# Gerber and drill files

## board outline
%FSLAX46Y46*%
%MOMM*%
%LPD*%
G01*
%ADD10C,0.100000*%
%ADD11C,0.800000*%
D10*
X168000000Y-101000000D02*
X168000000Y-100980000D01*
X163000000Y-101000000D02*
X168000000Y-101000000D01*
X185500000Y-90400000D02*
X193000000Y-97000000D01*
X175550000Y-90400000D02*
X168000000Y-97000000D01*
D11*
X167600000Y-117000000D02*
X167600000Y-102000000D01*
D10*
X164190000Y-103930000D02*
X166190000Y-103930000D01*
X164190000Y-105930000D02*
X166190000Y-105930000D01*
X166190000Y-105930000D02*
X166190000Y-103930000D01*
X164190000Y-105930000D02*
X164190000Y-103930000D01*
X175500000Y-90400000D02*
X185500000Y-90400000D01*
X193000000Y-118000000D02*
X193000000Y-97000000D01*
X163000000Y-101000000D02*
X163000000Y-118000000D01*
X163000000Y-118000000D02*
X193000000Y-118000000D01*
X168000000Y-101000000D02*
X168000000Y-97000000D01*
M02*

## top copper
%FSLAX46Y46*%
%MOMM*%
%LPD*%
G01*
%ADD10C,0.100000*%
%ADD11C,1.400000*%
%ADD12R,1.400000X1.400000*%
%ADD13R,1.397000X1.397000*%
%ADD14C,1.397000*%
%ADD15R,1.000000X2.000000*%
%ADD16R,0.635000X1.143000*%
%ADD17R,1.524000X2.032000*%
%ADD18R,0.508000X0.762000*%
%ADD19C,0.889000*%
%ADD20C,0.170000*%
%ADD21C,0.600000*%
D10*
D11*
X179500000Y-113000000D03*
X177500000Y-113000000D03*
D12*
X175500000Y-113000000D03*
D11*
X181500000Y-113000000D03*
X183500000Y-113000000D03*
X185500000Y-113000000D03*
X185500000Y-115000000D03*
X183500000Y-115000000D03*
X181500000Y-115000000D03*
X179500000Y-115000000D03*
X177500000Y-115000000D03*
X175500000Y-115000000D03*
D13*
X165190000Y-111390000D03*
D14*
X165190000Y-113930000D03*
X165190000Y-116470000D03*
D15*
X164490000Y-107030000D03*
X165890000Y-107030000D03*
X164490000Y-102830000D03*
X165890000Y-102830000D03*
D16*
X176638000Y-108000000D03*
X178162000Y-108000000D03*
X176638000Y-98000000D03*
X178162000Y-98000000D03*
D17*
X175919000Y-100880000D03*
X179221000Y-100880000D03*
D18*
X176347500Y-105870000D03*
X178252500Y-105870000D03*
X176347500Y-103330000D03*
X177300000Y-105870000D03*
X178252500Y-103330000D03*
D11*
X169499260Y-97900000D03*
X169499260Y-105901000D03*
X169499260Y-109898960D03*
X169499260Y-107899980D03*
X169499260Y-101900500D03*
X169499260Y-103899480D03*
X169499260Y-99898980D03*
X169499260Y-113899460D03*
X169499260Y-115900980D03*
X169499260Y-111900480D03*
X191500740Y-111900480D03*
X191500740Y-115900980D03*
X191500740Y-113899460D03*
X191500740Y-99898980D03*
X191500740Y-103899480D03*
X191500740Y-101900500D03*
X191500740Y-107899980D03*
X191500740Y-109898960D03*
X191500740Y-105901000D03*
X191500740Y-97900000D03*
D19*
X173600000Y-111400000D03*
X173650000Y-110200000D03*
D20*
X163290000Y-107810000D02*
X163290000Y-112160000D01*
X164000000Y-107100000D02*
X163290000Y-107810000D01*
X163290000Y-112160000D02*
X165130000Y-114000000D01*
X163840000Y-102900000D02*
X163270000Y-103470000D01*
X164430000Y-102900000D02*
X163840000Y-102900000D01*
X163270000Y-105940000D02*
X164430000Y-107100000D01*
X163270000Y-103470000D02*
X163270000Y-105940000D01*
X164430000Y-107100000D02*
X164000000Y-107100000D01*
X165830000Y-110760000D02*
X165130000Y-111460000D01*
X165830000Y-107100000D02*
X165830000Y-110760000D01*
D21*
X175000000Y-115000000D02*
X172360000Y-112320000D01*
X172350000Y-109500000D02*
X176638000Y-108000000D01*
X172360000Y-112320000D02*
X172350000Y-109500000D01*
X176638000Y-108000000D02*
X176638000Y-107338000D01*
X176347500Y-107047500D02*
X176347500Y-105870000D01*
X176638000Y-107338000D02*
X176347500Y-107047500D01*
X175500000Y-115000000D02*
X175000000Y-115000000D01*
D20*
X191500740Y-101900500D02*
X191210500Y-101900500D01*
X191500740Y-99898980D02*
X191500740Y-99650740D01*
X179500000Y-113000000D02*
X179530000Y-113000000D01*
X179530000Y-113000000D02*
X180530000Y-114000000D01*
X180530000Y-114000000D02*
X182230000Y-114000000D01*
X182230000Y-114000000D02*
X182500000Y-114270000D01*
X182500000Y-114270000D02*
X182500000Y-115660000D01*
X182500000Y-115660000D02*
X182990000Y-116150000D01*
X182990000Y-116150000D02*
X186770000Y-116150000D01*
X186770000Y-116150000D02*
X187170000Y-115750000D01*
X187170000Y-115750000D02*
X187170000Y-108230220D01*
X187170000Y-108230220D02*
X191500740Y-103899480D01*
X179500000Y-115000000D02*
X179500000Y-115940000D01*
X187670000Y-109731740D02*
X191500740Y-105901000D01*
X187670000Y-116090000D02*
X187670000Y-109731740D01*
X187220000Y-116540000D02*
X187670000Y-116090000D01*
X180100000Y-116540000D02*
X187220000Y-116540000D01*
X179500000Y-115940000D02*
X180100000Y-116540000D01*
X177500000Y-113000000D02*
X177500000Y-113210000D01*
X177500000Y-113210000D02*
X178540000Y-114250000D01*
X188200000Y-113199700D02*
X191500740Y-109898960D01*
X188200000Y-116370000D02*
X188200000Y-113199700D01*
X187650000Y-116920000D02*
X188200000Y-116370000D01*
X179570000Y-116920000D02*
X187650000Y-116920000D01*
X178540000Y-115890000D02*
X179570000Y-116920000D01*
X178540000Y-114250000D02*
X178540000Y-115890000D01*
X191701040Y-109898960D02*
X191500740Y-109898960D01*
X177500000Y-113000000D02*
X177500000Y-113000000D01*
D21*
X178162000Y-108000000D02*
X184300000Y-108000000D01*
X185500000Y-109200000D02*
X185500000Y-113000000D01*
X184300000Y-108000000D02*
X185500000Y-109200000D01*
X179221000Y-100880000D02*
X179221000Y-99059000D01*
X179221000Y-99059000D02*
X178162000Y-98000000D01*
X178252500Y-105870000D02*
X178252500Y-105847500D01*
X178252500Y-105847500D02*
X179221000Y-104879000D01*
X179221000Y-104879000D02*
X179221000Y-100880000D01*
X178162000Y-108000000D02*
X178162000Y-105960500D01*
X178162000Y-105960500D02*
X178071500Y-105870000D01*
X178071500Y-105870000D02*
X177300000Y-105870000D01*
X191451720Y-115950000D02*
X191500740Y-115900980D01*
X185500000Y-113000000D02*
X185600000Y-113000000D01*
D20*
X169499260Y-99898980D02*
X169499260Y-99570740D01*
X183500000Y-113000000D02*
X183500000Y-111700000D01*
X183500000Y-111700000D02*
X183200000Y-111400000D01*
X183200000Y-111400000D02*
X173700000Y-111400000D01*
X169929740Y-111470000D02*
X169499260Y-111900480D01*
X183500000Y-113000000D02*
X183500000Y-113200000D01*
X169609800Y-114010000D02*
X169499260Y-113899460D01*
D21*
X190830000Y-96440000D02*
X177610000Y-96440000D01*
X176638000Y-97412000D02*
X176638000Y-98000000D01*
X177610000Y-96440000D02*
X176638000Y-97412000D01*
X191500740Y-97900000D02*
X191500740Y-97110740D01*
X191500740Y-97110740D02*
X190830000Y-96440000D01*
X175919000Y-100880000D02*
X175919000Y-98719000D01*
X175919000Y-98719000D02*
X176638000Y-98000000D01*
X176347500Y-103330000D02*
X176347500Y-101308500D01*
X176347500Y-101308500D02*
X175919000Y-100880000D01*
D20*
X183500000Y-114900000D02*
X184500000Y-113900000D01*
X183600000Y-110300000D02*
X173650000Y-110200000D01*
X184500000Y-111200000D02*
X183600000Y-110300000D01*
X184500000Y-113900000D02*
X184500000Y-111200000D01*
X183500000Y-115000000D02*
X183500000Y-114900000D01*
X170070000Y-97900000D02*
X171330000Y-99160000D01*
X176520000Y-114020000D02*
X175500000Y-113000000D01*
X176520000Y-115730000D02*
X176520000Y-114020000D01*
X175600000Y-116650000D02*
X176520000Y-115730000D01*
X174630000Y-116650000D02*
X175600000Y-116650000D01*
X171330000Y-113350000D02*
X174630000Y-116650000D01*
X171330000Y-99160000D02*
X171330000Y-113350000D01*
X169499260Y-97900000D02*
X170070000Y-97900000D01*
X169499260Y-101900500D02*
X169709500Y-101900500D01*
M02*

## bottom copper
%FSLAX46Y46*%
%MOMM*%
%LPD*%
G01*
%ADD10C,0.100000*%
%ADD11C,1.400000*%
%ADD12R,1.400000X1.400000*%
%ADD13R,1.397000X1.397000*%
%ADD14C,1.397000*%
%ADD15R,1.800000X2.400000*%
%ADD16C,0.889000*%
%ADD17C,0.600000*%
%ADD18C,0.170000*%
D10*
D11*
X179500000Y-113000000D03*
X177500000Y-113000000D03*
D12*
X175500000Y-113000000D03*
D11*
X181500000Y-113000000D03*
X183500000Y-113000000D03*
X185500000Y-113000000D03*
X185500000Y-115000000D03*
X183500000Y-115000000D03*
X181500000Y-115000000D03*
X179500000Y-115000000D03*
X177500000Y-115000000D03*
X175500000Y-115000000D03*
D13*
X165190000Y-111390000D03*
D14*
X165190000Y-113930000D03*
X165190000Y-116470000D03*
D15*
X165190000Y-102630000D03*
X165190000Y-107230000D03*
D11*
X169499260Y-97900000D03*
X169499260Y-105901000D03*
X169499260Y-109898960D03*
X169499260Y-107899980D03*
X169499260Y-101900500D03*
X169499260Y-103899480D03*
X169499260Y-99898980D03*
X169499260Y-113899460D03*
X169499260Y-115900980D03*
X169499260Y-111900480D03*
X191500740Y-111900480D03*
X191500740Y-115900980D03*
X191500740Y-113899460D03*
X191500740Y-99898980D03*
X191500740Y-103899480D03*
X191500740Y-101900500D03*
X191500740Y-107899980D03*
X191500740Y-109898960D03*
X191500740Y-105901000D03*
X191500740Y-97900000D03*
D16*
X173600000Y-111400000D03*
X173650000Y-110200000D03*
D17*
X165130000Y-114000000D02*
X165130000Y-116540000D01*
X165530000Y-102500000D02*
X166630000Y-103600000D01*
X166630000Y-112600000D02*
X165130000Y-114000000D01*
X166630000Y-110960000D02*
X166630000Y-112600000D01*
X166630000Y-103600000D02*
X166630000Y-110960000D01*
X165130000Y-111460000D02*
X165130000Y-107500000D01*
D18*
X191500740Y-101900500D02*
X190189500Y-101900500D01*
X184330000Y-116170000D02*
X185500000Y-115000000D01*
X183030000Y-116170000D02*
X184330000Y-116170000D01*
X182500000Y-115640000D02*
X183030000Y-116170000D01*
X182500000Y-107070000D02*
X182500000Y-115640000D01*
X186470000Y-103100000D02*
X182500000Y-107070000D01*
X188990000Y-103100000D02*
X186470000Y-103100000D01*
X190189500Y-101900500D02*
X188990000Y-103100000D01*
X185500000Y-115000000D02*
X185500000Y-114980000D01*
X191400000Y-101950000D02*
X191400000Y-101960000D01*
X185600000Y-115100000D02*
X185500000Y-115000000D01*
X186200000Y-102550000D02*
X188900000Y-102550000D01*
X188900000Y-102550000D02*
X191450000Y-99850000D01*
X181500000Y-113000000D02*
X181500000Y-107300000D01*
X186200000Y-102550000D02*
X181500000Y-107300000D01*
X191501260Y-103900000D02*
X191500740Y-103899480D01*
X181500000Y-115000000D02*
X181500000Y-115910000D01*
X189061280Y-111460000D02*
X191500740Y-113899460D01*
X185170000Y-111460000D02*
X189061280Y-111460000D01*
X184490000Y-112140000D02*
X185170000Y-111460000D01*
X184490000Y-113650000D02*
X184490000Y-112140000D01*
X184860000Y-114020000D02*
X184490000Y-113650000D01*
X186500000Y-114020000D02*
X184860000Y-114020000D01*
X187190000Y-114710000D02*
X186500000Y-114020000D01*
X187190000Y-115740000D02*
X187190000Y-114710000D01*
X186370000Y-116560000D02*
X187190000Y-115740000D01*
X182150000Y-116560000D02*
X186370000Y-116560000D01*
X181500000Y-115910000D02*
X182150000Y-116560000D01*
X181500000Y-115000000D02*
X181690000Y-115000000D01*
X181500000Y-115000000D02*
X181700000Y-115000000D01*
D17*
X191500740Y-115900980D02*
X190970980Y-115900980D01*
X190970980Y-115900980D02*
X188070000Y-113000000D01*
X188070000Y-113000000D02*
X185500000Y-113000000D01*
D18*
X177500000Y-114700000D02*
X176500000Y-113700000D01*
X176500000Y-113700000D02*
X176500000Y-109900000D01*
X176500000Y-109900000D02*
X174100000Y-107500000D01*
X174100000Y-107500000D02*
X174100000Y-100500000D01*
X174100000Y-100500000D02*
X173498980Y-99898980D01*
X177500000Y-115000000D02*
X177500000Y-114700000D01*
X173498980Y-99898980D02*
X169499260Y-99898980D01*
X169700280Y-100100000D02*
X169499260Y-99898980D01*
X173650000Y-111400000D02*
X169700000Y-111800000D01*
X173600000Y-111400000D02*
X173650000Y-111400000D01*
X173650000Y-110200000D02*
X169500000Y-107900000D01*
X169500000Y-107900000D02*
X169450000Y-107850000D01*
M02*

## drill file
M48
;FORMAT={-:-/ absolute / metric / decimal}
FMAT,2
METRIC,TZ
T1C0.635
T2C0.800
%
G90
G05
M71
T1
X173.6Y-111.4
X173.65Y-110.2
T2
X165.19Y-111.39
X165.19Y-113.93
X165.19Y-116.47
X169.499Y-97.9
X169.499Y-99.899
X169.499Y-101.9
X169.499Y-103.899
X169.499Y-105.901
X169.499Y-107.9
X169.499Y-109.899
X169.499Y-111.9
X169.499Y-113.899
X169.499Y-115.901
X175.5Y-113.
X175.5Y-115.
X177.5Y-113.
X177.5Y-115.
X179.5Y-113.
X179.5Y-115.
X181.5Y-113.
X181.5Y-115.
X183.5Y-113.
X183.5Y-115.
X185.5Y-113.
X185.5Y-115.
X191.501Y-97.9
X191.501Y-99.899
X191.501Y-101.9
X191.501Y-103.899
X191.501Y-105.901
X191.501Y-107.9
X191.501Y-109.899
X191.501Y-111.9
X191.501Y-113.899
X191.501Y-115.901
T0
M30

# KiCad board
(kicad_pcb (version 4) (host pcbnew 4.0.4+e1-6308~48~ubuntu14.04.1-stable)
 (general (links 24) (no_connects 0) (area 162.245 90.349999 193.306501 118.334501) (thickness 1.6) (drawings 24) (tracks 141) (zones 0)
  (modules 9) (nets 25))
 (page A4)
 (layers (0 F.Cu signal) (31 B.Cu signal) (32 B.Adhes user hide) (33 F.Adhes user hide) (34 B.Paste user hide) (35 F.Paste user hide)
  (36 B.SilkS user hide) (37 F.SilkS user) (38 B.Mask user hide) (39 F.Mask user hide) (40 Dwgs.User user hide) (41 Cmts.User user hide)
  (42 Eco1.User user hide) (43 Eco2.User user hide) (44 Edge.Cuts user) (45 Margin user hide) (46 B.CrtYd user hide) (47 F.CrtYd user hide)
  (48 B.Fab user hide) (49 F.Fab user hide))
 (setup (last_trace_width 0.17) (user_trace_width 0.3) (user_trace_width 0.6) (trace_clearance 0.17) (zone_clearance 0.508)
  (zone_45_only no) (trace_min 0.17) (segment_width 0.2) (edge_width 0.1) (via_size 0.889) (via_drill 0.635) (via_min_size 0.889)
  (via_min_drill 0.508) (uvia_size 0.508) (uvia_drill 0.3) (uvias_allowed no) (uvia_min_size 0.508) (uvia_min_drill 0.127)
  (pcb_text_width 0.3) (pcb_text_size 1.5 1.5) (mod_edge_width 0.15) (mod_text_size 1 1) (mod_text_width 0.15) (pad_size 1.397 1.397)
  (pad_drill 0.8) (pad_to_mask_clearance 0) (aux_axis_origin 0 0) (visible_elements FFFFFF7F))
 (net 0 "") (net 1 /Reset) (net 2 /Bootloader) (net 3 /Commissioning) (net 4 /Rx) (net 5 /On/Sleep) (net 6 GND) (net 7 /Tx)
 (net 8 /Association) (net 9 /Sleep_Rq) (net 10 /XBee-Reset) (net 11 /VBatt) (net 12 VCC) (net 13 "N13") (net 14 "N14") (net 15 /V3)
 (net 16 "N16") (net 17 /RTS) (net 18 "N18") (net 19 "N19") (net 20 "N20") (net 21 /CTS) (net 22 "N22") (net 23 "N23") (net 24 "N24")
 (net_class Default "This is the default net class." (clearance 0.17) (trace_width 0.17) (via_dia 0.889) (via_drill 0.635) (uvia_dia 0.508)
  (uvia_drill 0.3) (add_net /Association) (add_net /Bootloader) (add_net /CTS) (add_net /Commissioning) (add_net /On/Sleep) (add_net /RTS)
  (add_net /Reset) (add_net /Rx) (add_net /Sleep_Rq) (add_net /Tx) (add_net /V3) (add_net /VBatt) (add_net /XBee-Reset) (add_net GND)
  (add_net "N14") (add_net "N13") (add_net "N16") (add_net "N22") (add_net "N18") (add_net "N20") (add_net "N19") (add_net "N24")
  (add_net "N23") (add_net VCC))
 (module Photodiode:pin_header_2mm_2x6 (layer B.Cu) (at 180.5 114)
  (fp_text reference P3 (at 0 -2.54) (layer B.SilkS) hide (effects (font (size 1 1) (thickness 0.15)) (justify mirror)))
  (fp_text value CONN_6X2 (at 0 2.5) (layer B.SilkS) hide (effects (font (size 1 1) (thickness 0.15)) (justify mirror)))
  (pad 5 thru_hole circle (at -1 -1) (size 1.4 1.4) (drill 0.8) (layers *.Cu *.Mask B.SilkS) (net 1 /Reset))
  (pad 3 thru_hole circle (at -3 -1) (size 1.4 1.4) (drill 0.8) (layers *.Cu *.Mask B.SilkS) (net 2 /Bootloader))
  (pad 1 thru_hole rect (at -5 -1) (size 1.4 1.4) (drill 0.8) (layers *.Cu *.Mask B.SilkS) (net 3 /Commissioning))
  (pad 7 thru_hole circle (at 1 -1) (size 1.4 1.4) (drill 0.8) (layers *.Cu *.Mask B.SilkS) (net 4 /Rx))
  (pad 9 thru_hole circle (at 3 -1) (size 1.4 1.4) (drill 0.8) (layers *.Cu *.Mask B.SilkS) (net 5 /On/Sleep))
  (pad 11 thru_hole circle (at 5 -1) (size 1.4 1.4) (drill 0.8) (layers *.Cu *.Mask B.SilkS) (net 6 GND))
  (pad 12 thru_hole circle (at 5 1) (size 1.4 1.4) (drill 0.8) (layers *.Cu *.Mask B.SilkS) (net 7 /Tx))
  (pad 10 thru_hole circle (at 3 1) (size 1.4 1.4) (drill 0.8) (layers *.Cu *.Mask B.SilkS) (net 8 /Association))
  (pad 8 thru_hole circle (at 1 1) (size 1.4 1.4) (drill 0.8) (layers *.Cu *.Mask B.SilkS) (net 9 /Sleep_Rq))
  (pad 6 thru_hole circle (at -1 1) (size 1.4 1.4) (drill 0.8) (layers *.Cu *.Mask B.SilkS) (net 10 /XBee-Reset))
  (pad 4 thru_hole circle (at -3 1) (size 1.4 1.4) (drill 0.8) (layers *.Cu *.Mask B.SilkS) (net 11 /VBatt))
  (pad 2 thru_hole circle (at -5 1) (size 1.4 1.4) (drill 0.8) (layers *.Cu *.Mask B.SilkS) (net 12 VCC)))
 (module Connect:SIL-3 (layer F.Cu) (at 165.19 113.93 270)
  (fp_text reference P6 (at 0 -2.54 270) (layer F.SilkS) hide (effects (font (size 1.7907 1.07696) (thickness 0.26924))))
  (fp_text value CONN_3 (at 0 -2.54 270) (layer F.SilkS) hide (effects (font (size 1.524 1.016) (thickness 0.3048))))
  (pad 1 thru_hole rect (at -2.54 0 270) (size 1.397 1.397) (drill 0.8) (layers *.Cu *.Mask F.SilkS) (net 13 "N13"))
  (pad 2 thru_hole circle (at 0 0 270) (size 1.397 1.397) (drill 0.8) (layers *.Cu *.Mask F.SilkS) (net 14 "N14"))
  (pad 3 thru_hole circle (at 2.54 0 270) (size 1.397 1.397) (drill 0.8) (layers *.Cu *.Mask F.SilkS) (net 14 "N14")))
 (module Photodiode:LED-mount (layer F.Cu) (at 165.19 104.83 90)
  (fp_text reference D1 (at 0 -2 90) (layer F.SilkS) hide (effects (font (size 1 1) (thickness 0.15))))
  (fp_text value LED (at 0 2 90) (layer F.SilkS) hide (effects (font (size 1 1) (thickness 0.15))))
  (pad 1 smd rect (at 2.2 0 90) (size 2.4 1.8) (layers B.Cu F.Paste B.Mask) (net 14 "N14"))
  (pad 2 smd rect (at -2.4 0 90) (size 2.4 1.8) (layers B.Cu F.Paste B.Mask) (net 13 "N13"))
  (pad 3 smd rect (at -2.2 -0.7 90) (size 2 1) (layers F.Cu F.Paste F.Mask))
  (pad 4 smd rect (at -2.2 0.7 90) (size 2 1) (layers F.Cu F.Paste F.Mask))
  (pad 5 smd rect (at 2 -0.7 90) (size 2 1) (layers F.Cu F.Paste F.Mask))
  (pad 6 smd rect (at 2 0.7 90) (size 2 1) (layers F.Cu F.Paste F.Mask)))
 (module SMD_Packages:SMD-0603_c (layer F.Cu) (at 177.4 108)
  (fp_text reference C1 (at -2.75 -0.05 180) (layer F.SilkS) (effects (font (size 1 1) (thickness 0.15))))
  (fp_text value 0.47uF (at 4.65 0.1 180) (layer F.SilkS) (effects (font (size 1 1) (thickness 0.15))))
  (pad 1 smd rect (at -0.762 0) (size 0.635 1.143) (layers F.Cu F.Paste F.Mask) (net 12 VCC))
  (pad 2 smd rect (at 0.762 0) (size 0.635 1.143) (layers F.Cu F.Paste F.Mask) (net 6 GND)))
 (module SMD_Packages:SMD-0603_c (layer F.Cu) (at 177.4 98)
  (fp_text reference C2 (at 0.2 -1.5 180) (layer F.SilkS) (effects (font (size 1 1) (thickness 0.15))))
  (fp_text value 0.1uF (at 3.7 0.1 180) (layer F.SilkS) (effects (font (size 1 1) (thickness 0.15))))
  (pad 1 smd rect (at -0.762 0) (size 0.635 1.143) (layers F.Cu F.Paste F.Mask) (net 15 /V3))
  (pad 2 smd rect (at 0.762 0) (size 0.635 1.143) (layers F.Cu F.Paste F.Mask) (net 6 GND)))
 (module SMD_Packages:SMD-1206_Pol (layer F.Cu) (at 177.57 100.88)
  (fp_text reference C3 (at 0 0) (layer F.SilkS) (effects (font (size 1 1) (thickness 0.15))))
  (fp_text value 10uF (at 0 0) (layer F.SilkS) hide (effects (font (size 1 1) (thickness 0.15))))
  (pad 1 smd rect (at -1.651 0) (size 1.524 2.032) (layers F.Cu F.Paste F.Mask) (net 15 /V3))
  (pad 2 smd rect (at 1.651 0) (size 1.524 2.032) (layers F.Cu F.Paste F.Mask) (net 6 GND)))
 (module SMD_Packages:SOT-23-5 (layer F.Cu) (at 177.3 104.6)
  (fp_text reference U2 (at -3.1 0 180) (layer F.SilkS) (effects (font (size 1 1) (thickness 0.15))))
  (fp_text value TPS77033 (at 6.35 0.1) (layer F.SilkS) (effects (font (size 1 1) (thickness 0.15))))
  (pad 1 smd rect (at -0.9525 1.27) (size 0.508 0.762) (layers F.Cu F.Paste F.Mask) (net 12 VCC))
  (pad 3 smd rect (at 0.9525 1.27) (size 0.508 0.762) (layers F.Cu F.Paste F.Mask) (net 6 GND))
  (pad 5 smd rect (at -0.9525 -1.27) (size 0.508 0.762) (layers F.Cu F.Paste F.Mask) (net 15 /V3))
  (pad 2 smd rect (at 0 1.27) (size 0.508 0.762) (layers F.Cu F.Paste F.Mask) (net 6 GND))
  (pad 4 smd rect (at 0.9525 -1.27) (size 0.508 0.762) (layers F.Cu F.Paste F.Mask) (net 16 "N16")))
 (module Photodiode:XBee (layer B.Cu) (at 180.5 97.9 180)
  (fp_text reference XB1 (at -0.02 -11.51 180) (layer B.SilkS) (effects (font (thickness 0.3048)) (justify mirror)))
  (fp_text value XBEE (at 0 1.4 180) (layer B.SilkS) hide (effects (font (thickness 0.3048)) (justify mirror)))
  (pad 20 thru_hole circle (at 11.00074 0 180) (size 1.4 1.4) (drill 0.8) (layers *.Cu *.Mask) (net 3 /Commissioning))
  (pad 16 thru_hole circle (at 11.00074 -8.001 180) (size 1.4 1.4) (drill 0.8) (layers *.Cu *.Mask) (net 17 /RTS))
  (pad 14 thru_hole circle (at 11.00074 -11.99896 180) (size 1.4 1.4) (drill 0.8) (layers *.Cu *.Mask) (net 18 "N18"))
  (pad 15 thru_hole circle (at 11.00074 -9.99998 180) (size 1.4 1.4) (drill 0.8) (layers *.Cu *.Mask) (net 8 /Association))
  (pad 18 thru_hole circle (at 11.00074 -4.0005 180) (size 1.4 1.4) (drill 0.8) (layers *.Cu *.Mask) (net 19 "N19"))
  (pad 17 thru_hole circle (at 11.00074 -5.99948 180) (size 1.4 1.4) (drill 0.8) (layers *.Cu *.Mask) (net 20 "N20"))
  (pad 19 thru_hole circle (at 11.00074 -1.99898 180) (size 1.4 1.4) (drill 0.8) (layers *.Cu *.Mask) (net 11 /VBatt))
  (pad 12 thru_hole circle (at 11.00074 -15.99946 180) (size 1.4 1.4) (drill 0.8) (layers *.Cu *.Mask) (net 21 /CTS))
  (pad 11 thru_hole circle (at 11.00074 -18.00098 180) (size 1.4 1.4) (drill 0.8) (layers *.Cu *.Mask) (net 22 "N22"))
  (pad 13 thru_hole circle (at 11.00074 -14.00048 180) (size 1.4 1.4) (drill 0.8) (layers *.Cu *.Mask) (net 5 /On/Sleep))
  (pad 8 thru_hole circle (at -11.00074 -14.00048 180) (size 1.4 1.4) (drill 0.8) (layers *.Cu *.Mask) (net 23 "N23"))
  (pad 10 thru_hole circle (at -11.00074 -18.00098 180) (size 1.4 1.4) (drill 0.8) (layers *.Cu *.Mask) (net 6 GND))
  (pad 9 thru_hole circle (at -11.00074 -15.99946 180) (size 1.4 1.4) (drill 0.8) (layers *.Cu *.Mask) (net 9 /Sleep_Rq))
  (pad 2 thru_hole circle (at -11.00074 -1.99898 180) (size 1.4 1.4) (drill 0.8) (layers *.Cu *.Mask) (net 4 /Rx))
  (pad 4 thru_hole circle (at -11.00074 -5.99948 180) (size 1.4 1.4) (drill 0.8) (layers *.Cu *.Mask) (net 1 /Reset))
  (pad 3 thru_hole circle (at -11.00074 -4.0005 180) (size 1.4 1.4) (drill 0.8) (layers *.Cu *.Mask) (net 7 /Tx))
  (pad 6 thru_hole circle (at -11.00074 -9.99998 180) (size 1.4 1.4) (drill 0.8) (layers *.Cu *.Mask) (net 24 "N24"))
  (pad 7 thru_hole circle (at -11.00074 -11.99896 180) (size 1.4 1.4) (drill 0.8) (layers *.Cu *.Mask) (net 2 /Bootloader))
  (pad 5 thru_hole circle (at -11.00074 -8.001 180) (size 1.4 1.4) (drill 0.8) (layers *.Cu *.Mask) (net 10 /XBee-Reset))
  (pad 1 thru_hole circle (at -11.00074 0 180) (size 1.4 1.4) (drill 0.8) (layers *.Cu *.Mask) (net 15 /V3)))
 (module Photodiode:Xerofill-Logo (layer F.Cu) (at 180.34 94.25)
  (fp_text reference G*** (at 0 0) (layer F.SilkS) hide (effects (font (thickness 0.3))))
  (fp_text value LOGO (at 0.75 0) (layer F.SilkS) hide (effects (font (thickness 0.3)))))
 (gr_line (start 168 101) (end 168 100.98) (angle 90) (layer Edge.Cuts) (width 0.1))
 (gr_line (start 163 101) (end 168 101) (angle 90) (layer Edge.Cuts) (width 0.1))
 (gr_line (start 185.5 90.4) (end 193 97) (angle 90) (layer Edge.Cuts) (width 0.1))
 (gr_line (start 175.55 90.4) (end 168 97) (angle 90) (layer Edge.Cuts) (width 0.1))
 (gr_line (start 167.6 117) (end 167.6 102) (angle 90) (layer Edge.Cuts) (width 0.8))
 (gr_line (start 164.19 103.93) (end 166.19 103.93) (angle 90) (layer Edge.Cuts) (width 0.1))
 (gr_line (start 164.19 105.93) (end 166.19 105.93) (angle 90) (layer Edge.Cuts) (width 0.1))
 (gr_line (start 166.19 105.93) (end 166.19 103.93) (angle 90) (layer Edge.Cuts) (width 0.1))
 (gr_line (start 164.19 105.93) (end 164.19 103.93) (angle 90) (layer Edge.Cuts) (width 0.1))
 (gr_line (start 175.5 90.4) (end 185.5 90.4) (angle 90) (layer Edge.Cuts) (width 0.1))
 (gr_line (start 193 118) (end 193 97) (angle 90) (layer Edge.Cuts) (width 0.1))
 (gr_line (start 163 101) (end 163 118) (angle 90) (layer Edge.Cuts) (width 0.1))
 (gr_line (start 163 118) (end 193 118) (angle 90) (layer Edge.Cuts) (width 0.1))
 (gr_line (start 168 101) (end 168 97) (angle 90) (layer Edge.Cuts) (width 0.1))
 (segment (start 163.29 107.81) (end 163.29 112.16) (width 0.17) (layer F.Cu) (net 14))
 (segment (start 164 107.1) (end 163.29 107.81) (width 0.17) (layer F.Cu) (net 14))
 (segment (start 165.13 114) (end 165.13 116.54) (width 0.6) (layer B.Cu) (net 14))
 (segment (start 165.53 102.5) (end 166.63 103.6) (width 0.6) (layer B.Cu) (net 14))
 (segment (start 166.63 112.6) (end 165.13 114) (width 0.6) (layer B.Cu) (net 14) (status 20))
 (segment (start 163.29 112.16) (end 165.13 114) (width 0.17) (layer F.Cu) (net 14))
 (segment (start 166.63 110.96) (end 166.63 112.6) (width 0.6) (layer B.Cu) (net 14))
 (segment (start 163.84 102.9) (end 163.27 103.47) (width 0.17) (layer F.Cu) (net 14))
 (segment (start 164.43 102.9) (end 163.84 102.9) (width 0.17) (layer F.Cu) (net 14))
 (segment (start 163.27 105.94) (end 164.43 107.1) (width 0.17) (layer F.Cu) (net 14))
 (segment (start 163.27 103.47) (end 163.27 105.94) (width 0.17) (layer F.Cu) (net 14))
 (segment (start 164.43 107.1) (end 164 107.1) (width 0.17) (layer F.Cu) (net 14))
 (segment (start 166.63 103.6) (end 166.63 110.96) (width 0.6) (layer B.Cu) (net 14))
 (segment (start 165.83 110.76) (end 165.13 111.46) (width 0.17) (layer F.Cu) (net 13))
 (segment (start 165.83 107.1) (end 165.83 110.76) (width 0.17) (layer F.Cu) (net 13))
 (segment (start 165.13 111.46) (end 165.13 107.5) (width 0.6) (layer B.Cu) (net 13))
 (segment (start 175 115) (end 172.36 112.32) (width 0.6) (layer F.Cu) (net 12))
 (segment (start 172.35 109.5) (end 176.638 108) (width 0.6) (layer F.Cu) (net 12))
 (segment (start 172.36 112.32) (end 172.35 109.5) (width 0.6) (layer F.Cu) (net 12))
 (segment (start 176.638 108) (end 176.638 107.338) (width 0.6) (layer F.Cu) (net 12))
 (segment (start 176.3475 107.0475) (end 176.3475 105.87) (width 0.6) (layer F.Cu) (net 12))
 (segment (start 176.638 107.338) (end 176.3475 107.0475) (width 0.6) (layer F.Cu) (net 12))
 (segment (start 175.5 115) (end 175 115) (width 0.6) (layer F.Cu) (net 12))
 (segment (start 191.50074 101.9005) (end 190.1895 101.9005) (width 0.17) (layer B.Cu) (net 7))
 (segment (start 184.33 116.17) (end 185.5 115) (width 0.17) (layer B.Cu) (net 7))
 (segment (start 183.03 116.17) (end 184.33 116.17) (width 0.17) (layer B.Cu) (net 7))
 (segment (start 182.5 115.64) (end 183.03 116.17) (width 0.17) (layer B.Cu) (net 7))
 (segment (start 182.5 107.07) (end 182.5 115.64) (width 0.17) (layer B.Cu) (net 7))
 (segment (start 186.47 103.1) (end 182.5 107.07) (width 0.17) (layer B.Cu) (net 7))
 (segment (start 188.99 103.1) (end 186.47 103.1) (width 0.17) (layer B.Cu) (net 7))
 (segment (start 190.1895 101.9005) (end 188.99 103.1) (width 0.17) (layer B.Cu) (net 7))
 (segment (start 185.5 115) (end 185.5 114.98) (width 0.17) (layer B.Cu) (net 7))
 (segment (start 191.50074 101.9005) (end 191.2105 101.9005) (width 0.17) (layer F.Cu) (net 7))
 (segment (start 191.4 101.95) (end 191.4 101.96) (width 0.17) (layer B.Cu) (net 7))
 (segment (start 185.6 115.1) (end 185.5 115) (width 0.17) (layer B.Cu) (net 7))
 (segment (start 191.50074 99.89898) (end 191.50074 99.65074) (width 0.17) (layer F.Cu) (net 4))
 (segment (start 186.2 102.55) (end 188.9 102.55) (width 0.17) (layer B.Cu) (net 4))
 (segment (start 188.9 102.55) (end 191.45 99.85) (width 0.17) (layer B.Cu) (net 4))
 (segment (start 181.5 113) (end 181.5 107.3) (width 0.17) (layer B.Cu) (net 4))
 (segment (start 186.2 102.55) (end 181.5 107.3) (width 0.17) (layer B.Cu) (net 4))
 (segment (start 179.5 113) (end 179.53 113) (width 0.17) (layer F.Cu) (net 1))
 (segment (start 179.53 113) (end 180.53 114) (width 0.17) (layer F.Cu) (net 1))
 (segment (start 180.53 114) (end 182.23 114) (width 0.17) (layer F.Cu) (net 1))
 (segment (start 182.23 114) (end 182.5 114.27) (width 0.17) (layer F.Cu) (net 1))
 (segment (start 182.5 114.27) (end 182.5 115.66) (width 0.17) (layer F.Cu) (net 1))
 (segment (start 182.5 115.66) (end 182.99 116.15) (width 0.17) (layer F.Cu) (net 1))
 (segment (start 182.99 116.15) (end 186.77 116.15) (width 0.17) (layer F.Cu) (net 1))
 (segment (start 186.77 116.15) (end 187.17 115.75) (width 0.17) (layer F.Cu) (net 1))
 (segment (start 187.17 115.75) (end 187.17 108.23022) (width 0.17) (layer F.Cu) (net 1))
 (segment (start 187.17 108.23022) (end 191.50074 103.89948) (width 0.17) (layer F.Cu) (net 1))
 (segment (start 191.50126 103.9) (end 191.50074 103.89948) (width 0.17) (layer B.Cu) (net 1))
 (segment (start 179.5 115) (end 179.5 115.94) (width 0.17) (layer F.Cu) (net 10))
 (segment (start 187.67 109.73174) (end 191.50074 105.901) (width 0.17) (layer F.Cu) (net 10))
 (segment (start 187.67 116.09) (end 187.67 109.73174) (width 0.17) (layer F.Cu) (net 10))
 (segment (start 187.22 116.54) (end 187.67 116.09) (width 0.17) (layer F.Cu) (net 10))
 (segment (start 180.1 116.54) (end 187.22 116.54) (width 0.17) (layer F.Cu) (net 10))
 (segment (start 179.5 115.94) (end 180.1 116.54) (width 0.17) (layer F.Cu) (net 10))
 (segment (start 177.5 113) (end 177.5 113.21) (width 0.17) (layer F.Cu) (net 2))
 (segment (start 177.5 113.21) (end 178.54 114.25) (width 0.17) (layer F.Cu) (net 2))
 (segment (start 188.2 113.1997) (end 191.50074 109.89896) (width 0.17) (layer F.Cu) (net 2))
 (segment (start 188.2 116.37) (end 188.2 113.1997) (width 0.17) (layer F.Cu) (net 2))
 (segment (start 187.65 116.92) (end 188.2 116.37) (width 0.17) (layer F.Cu) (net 2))
 (segment (start 179.57 116.92) (end 187.65 116.92) (width 0.17) (layer F.Cu) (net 2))
 (segment (start 178.54 115.89) (end 179.57 116.92) (width 0.17) (layer F.Cu) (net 2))
 (segment (start 178.54 114.25) (end 178.54 115.89) (width 0.17) (layer F.Cu) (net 2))
 (segment (start 191.70104 109.89896) (end 191.50074 109.89896) (width 0.17) (layer F.Cu) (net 2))
 (segment (start 177.5 113) (end 177.5 113) (width 0.17) (layer F.Cu) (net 2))
 (segment (start 181.5 115) (end 181.5 115.91) (width 0.17) (layer B.Cu) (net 9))
 (segment (start 189.06128 111.46) (end 191.50074 113.89946) (width 0.17) (layer B.Cu) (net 9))
 (segment (start 185.17 111.46) (end 189.06128 111.46) (width 0.17) (layer B.Cu) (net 9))
 (segment (start 184.49 112.14) (end 185.17 111.46) (width 0.17) (layer B.Cu) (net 9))
 (segment (start 184.49 113.65) (end 184.49 112.14) (width 0.17) (layer B.Cu) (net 9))
 (segment (start 184.86 114.02) (end 184.49 113.65) (width 0.17) (layer B.Cu) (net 9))
 (segment (start 186.5 114.02) (end 184.86 114.02) (width 0.17) (layer B.Cu) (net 9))
 (segment (start 187.19 114.71) (end 186.5 114.02) (width 0.17) (layer B.Cu) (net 9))
 (segment (start 187.19 115.74) (end 187.19 114.71) (width 0.17) (layer B.Cu) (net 9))
 (segment (start 186.37 116.56) (end 187.19 115.74) (width 0.17) (layer B.Cu) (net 9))
 (segment (start 182.15 116.56) (end 186.37 116.56) (width 0.17) (layer B.Cu) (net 9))
 (segment (start 181.5 115.91) (end 182.15 116.56) (width 0.17) (layer B.Cu) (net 9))
 (segment (start 181.5 115) (end 181.69 115) (width 0.17) (layer B.Cu) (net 9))
 (segment (start 181.5 115) (end 181.7 115) (width 0.17) (layer B.Cu) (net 9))
 (segment (start 191.50074 115.90098) (end 190.97098 115.90098) (width 0.6) (layer B.Cu) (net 6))
 (segment (start 190.97098 115.90098) (end 188.07 113) (width 0.6) (layer B.Cu) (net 6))
 (segment (start 188.07 113) (end 185.5 113) (width 0.6) (layer B.Cu) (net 6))
 (segment (start 178.162 108) (end 184.3 108) (width 0.6) (layer F.Cu) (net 6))
 (segment (start 185.5 109.2) (end 185.5 113) (width 0.6) (layer F.Cu) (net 6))
 (segment (start 184.3 108) (end 185.5 109.2) (width 0.6) (layer F.Cu) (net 6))
 (segment (start 179.221 100.88) (end 179.221 99.059) (width 0.6) (layer F.Cu) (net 6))
 (segment (start 179.221 99.059) (end 178.162 98) (width 0.6) (layer F.Cu) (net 6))
 (segment (start 178.2525 105.87) (end 178.2525 105.8475) (width 0.6) (layer F.Cu) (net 6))
 (segment (start 178.2525 105.8475) (end 179.221 104.879) (width 0.6) (layer F.Cu) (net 6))
 (segment (start 179.221 104.879) (end 179.221 100.88) (width 0.6) (layer F.Cu) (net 6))
 (segment (start 178.162 108) (end 178.162 105.9605) (width 0.6) (layer F.Cu) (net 6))
 (segment (start 178.162 105.9605) (end 178.0715 105.87) (width 0.6) (layer F.Cu) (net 6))
 (segment (start 178.0715 105.87) (end 177.3 105.87) (width 0.6) (layer F.Cu) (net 6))
 (segment (start 191.45172 115.95) (end 191.50074 115.90098) (width 0.6) (layer F.Cu) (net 6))
 (segment (start 185.5 113) (end 185.6 113) (width 0.6) (layer F.Cu) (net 6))
 (segment (start 177.5 114.7) (end 176.5 113.7) (width 0.17) (layer B.Cu) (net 11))
 (segment (start 176.5 113.7) (end 176.5 109.9) (width 0.17) (layer B.Cu) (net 11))
 (segment (start 176.5 109.9) (end 174.1 107.5) (width 0.17) (layer B.Cu) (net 11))
 (segment (start 174.1 107.5) (end 174.1 100.5) (width 0.17) (layer B.Cu) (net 11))
 (segment (start 174.1 100.5) (end 173.49898 99.89898) (width 0.17) (layer B.Cu) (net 11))
 (segment (start 169.49926 99.89898) (end 169.49926 99.57074) (width 0.17) (layer F.Cu) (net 11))
 (segment (start 177.5 115) (end 177.5 114.7) (width 0.17) (layer B.Cu) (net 11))
 (segment (start 173.49898 99.89898) (end 169.49926 99.89898) (width 0.17) (layer B.Cu) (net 11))
 (segment (start 169.70028 100.1) (end 169.49926 99.89898) (width 0.17) (layer B.Cu) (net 11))
 (segment (start 183.5 113) (end 183.5 111.7) (width 0.17) (layer F.Cu) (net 5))
 (segment (start 183.5 111.7) (end 183.2 111.4) (width 0.17) (layer F.Cu) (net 5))
 (segment (start 183.2 111.4) (end 173.7 111.4) (width 0.17) (layer F.Cu) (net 5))
 (via (at 173.6 111.4) (size 0.889) (drill 0.635) (layers F.Cu B.Cu) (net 5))
 (segment (start 173.65 111.4) (end 169.7 111.8) (width 0.17) (layer B.Cu) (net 5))
 (segment (start 173.6 111.4) (end 173.65 111.4) (width 0.17) (layer B.Cu) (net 5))
 (segment (start 169.92974 111.47) (end 169.49926 111.90048) (width 0.17) (layer F.Cu) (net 5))
 (segment (start 183.5 113) (end 183.5 113.2) (width 0.17) (layer F.Cu) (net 5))
 (segment (start 169.6098 114.01) (end 169.49926 113.89946) (width 0.17) (layer F.Cu) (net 21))
 (segment (start 190.83 96.44) (end 177.61 96.44) (width 0.6) (layer F.Cu) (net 15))
 (segment (start 176.638 97.412) (end 176.638 98) (width 0.6) (layer F.Cu) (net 15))
 (segment (start 177.61 96.44) (end 176.638 97.412) (width 0.6) (layer F.Cu) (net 15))
 (segment (start 191.50074 97.9) (end 191.50074 97.11074) (width 0.6) (layer F.Cu) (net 15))
 (segment (start 191.50074 97.11074) (end 190.83 96.44) (width 0.6) (layer F.Cu) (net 15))
 (segment (start 175.919 100.88) (end 175.919 98.719) (width 0.6) (layer F.Cu) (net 15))
 (segment (start 175.919 98.719) (end 176.638 98) (width 0.6) (layer F.Cu) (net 15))
 (segment (start 176.3475 103.33) (end 176.3475 101.3085) (width 0.6) (layer F.Cu) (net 15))
 (segment (start 176.3475 101.3085) (end 175.919 100.88) (width 0.6) (layer F.Cu) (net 15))
 (segment (start 183.5 114.9) (end 184.5 113.9) (width 0.17) (layer F.Cu) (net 8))
 (segment (start 173.65 110.2) (end 169.5 107.9) (width 0.17) (layer B.Cu) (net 8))
 (via (at 173.65 110.2) (size 0.889) (drill 0.635) (layers F.Cu B.Cu) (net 8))
 (segment (start 183.6 110.3) (end 173.65 110.2) (width 0.17) (layer F.Cu) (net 8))
 (segment (start 184.5 111.2) (end 183.6 110.3) (width 0.17) (layer F.Cu) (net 8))
 (segment (start 184.5 113.9) (end 184.5 111.2) (width 0.17) (layer F.Cu) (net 8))
 (segment (start 183.5 115) (end 183.5 114.9) (width 0.17) (layer F.Cu) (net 8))
 (segment (start 169.5 107.9) (end 169.45 107.85) (width 0.17) (layer B.Cu) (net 8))
 (segment (start 170.07 97.9) (end 171.33 99.16) (width 0.17) (layer F.Cu) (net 3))
 (segment (start 176.52 114.02) (end 175.5 113) (width 0.17) (layer F.Cu) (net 3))
 (segment (start 176.52 115.73) (end 176.52 114.02) (width 0.17) (layer F.Cu) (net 3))
 (segment (start 175.6 116.65) (end 176.52 115.73) (width 0.17) (layer F.Cu) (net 3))
 (segment (start 174.63 116.65) (end 175.6 116.65) (width 0.17) (layer F.Cu) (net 3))
 (segment (start 171.33 113.35) (end 174.63 116.65) (width 0.17) (layer F.Cu) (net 3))
 (segment (start 171.33 99.16) (end 171.33 113.35) (width 0.17) (layer F.Cu) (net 3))
 (segment (start 169.49926 97.9) (end 170.07 97.9) (width 0.17) (layer F.Cu) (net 3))
 (segment (start 169.49926 101.9005) (end 169.7095 101.9005) (width 0.17) (layer F.Cu) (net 19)))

